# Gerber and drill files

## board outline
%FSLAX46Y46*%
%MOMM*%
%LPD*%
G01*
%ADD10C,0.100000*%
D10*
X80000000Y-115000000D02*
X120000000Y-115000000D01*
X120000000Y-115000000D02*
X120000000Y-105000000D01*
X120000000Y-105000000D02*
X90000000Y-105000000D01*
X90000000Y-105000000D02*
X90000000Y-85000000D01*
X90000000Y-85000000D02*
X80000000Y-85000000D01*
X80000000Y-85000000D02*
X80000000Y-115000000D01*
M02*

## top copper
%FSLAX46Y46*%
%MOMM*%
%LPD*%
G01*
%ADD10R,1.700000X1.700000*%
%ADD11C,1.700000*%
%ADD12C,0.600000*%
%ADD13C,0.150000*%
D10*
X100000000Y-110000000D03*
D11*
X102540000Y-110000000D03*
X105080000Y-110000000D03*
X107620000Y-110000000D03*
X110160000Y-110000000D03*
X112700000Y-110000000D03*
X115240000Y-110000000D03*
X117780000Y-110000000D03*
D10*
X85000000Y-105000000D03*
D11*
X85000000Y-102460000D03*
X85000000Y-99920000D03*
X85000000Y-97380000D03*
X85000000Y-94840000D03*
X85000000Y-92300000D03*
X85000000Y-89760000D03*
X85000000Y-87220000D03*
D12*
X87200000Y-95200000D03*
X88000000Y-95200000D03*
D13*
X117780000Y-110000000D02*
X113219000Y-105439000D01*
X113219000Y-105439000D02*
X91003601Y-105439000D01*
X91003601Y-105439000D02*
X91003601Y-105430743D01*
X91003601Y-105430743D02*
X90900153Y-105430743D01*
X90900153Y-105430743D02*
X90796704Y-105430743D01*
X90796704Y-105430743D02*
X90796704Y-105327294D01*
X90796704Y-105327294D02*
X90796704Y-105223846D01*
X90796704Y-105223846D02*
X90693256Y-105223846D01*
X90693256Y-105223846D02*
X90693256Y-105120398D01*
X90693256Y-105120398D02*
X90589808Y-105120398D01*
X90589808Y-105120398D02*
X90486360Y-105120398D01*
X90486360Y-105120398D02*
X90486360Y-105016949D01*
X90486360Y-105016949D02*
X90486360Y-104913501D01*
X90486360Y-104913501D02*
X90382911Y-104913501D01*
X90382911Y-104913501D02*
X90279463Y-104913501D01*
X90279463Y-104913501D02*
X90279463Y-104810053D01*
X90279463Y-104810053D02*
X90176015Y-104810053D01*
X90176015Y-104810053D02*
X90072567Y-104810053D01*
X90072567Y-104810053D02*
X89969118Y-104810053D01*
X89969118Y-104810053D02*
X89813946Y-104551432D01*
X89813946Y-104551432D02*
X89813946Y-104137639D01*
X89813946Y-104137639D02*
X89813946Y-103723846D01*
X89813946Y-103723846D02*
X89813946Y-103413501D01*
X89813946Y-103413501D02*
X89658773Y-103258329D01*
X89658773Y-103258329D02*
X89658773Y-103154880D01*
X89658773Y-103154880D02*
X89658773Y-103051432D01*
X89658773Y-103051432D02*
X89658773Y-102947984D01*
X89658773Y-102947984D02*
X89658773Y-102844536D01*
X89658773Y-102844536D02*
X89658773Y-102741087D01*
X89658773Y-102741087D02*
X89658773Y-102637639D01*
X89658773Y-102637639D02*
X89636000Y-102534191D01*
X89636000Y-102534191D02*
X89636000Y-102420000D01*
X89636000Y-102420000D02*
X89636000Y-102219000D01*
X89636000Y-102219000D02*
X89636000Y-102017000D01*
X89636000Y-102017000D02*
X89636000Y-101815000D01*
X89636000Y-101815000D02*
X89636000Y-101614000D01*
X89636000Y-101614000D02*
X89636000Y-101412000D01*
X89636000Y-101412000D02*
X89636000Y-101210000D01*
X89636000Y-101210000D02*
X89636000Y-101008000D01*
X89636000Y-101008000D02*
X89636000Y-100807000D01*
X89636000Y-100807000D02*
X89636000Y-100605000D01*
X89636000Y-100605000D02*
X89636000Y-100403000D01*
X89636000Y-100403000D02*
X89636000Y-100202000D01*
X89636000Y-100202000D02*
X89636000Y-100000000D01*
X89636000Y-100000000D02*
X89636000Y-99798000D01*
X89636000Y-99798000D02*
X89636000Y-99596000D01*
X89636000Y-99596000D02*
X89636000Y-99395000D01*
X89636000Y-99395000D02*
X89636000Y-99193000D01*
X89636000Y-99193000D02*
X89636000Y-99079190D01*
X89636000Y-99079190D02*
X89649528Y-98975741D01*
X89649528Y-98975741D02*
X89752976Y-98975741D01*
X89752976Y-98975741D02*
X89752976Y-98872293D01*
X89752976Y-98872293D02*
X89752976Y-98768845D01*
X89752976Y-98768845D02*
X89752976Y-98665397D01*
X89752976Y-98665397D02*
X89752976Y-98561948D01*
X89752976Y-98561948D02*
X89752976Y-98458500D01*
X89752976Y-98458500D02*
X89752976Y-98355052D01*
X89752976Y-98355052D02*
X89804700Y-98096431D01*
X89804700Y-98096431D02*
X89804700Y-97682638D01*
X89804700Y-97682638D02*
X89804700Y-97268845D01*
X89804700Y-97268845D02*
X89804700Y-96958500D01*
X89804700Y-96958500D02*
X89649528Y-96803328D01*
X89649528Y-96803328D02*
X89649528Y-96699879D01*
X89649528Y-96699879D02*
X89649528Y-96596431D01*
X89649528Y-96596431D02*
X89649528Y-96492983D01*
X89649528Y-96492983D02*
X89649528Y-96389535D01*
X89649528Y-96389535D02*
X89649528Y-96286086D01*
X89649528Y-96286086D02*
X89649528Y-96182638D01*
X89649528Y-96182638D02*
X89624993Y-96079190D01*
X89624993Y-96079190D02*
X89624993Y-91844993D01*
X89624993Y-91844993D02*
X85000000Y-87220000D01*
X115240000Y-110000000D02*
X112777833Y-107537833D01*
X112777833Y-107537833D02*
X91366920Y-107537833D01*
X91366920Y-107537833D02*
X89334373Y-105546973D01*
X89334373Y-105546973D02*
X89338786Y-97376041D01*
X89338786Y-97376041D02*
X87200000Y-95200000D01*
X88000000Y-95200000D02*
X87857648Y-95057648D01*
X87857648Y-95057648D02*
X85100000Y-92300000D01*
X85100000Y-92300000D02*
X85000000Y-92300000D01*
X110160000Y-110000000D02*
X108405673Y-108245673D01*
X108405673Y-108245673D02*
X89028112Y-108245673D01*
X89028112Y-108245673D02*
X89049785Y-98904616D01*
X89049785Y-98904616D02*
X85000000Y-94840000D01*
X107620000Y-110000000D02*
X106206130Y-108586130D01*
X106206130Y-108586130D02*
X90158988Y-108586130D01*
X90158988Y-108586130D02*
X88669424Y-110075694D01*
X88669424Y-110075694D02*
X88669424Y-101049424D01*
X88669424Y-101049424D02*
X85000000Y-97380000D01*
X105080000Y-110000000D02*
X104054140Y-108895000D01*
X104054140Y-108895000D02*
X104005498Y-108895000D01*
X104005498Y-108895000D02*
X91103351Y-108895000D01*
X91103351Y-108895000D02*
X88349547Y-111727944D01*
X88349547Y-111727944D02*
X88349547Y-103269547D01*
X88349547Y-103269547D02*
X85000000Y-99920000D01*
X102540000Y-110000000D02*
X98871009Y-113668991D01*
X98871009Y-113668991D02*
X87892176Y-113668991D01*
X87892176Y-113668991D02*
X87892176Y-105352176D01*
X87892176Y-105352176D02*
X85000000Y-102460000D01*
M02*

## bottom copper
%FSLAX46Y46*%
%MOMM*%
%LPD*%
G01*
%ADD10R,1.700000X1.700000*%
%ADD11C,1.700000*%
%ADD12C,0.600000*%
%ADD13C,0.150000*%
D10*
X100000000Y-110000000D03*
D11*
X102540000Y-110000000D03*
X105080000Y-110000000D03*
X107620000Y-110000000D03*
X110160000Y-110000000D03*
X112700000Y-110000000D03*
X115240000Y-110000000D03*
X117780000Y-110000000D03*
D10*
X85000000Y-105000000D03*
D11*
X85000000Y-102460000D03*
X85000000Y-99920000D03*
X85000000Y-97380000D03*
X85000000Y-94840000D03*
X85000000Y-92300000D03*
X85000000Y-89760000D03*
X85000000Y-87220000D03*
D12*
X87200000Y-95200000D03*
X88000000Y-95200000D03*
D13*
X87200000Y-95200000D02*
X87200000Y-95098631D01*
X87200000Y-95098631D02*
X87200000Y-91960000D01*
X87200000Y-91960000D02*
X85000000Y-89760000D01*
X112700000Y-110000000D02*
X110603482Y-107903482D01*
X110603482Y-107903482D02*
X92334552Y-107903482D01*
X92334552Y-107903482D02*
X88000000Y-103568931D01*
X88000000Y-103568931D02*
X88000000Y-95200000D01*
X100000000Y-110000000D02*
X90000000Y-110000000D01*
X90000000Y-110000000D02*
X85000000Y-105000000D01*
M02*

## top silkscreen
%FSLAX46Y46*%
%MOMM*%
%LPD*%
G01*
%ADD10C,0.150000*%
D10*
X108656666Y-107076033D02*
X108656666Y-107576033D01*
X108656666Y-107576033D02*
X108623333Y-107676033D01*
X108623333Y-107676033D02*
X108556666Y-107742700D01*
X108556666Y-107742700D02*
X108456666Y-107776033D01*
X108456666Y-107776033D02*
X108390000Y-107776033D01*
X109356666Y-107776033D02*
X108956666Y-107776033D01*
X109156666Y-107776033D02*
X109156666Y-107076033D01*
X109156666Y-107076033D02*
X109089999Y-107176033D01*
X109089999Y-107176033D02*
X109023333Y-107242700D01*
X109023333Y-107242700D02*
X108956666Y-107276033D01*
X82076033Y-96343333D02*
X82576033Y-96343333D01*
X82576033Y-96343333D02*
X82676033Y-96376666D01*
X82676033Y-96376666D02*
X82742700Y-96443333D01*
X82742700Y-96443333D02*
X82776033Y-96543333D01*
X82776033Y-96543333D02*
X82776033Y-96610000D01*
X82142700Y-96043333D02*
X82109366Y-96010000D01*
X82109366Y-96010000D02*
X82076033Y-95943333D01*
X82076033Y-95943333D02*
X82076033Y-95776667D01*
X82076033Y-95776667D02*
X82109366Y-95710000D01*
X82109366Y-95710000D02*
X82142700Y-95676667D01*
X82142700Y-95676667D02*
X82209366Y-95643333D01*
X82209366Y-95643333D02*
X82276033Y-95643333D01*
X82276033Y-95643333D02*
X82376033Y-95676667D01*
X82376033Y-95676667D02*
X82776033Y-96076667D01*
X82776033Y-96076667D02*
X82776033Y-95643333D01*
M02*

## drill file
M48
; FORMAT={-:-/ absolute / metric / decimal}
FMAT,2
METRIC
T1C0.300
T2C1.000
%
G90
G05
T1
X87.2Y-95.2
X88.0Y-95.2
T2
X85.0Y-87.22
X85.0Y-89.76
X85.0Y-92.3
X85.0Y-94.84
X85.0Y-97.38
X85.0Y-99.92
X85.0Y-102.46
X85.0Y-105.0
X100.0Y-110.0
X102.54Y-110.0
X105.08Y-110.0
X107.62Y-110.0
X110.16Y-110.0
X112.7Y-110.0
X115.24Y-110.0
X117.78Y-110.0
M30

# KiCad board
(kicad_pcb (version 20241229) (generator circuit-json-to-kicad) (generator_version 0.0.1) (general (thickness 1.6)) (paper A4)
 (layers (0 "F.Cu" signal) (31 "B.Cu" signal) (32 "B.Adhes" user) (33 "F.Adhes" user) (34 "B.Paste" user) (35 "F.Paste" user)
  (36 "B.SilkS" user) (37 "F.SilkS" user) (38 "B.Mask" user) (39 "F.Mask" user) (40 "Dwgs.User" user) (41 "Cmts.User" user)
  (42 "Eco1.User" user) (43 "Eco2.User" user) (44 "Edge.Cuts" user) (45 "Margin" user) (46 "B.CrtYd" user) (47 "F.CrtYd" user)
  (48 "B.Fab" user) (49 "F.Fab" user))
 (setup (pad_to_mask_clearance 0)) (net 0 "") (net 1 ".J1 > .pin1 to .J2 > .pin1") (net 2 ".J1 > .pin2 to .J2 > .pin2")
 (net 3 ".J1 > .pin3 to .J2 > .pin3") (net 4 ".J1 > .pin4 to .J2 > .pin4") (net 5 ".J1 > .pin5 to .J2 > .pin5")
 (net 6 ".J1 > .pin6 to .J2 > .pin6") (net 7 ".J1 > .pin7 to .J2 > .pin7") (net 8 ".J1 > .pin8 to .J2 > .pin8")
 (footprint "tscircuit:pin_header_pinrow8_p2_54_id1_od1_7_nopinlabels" (layer F.Cu) (at 108.89 110 0)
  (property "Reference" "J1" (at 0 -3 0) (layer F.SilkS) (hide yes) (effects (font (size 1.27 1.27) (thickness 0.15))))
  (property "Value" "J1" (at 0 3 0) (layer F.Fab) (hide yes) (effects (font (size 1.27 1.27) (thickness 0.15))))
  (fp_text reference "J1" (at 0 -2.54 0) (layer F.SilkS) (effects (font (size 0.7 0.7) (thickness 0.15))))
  (pad "1" thru_hole rect (at -8.89 0 0) (size 1.7 1.7) (drill 1) (layers *.Cu *.Mask) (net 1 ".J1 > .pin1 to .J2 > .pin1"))
  (pad "2" thru_hole circle (at -6.3500000000000005 0 0) (size 1.7 1.7) (drill 1) (layers *.Cu *.Mask) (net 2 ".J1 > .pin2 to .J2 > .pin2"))
  (pad "3" thru_hole circle (at -3.8100000000000005 0 0) (size 1.7 1.7) (drill 1) (layers *.Cu *.Mask) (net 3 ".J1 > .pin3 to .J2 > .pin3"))
  (pad "4" thru_hole circle (at -1.2700000000000005 0 0) (size 1.7 1.7) (drill 1) (layers *.Cu *.Mask) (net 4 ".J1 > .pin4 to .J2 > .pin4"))
  (pad "5" thru_hole circle (at 1.2699999999999996 0 0) (size 1.7 1.7) (drill 1) (layers *.Cu *.Mask) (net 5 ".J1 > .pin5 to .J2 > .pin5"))
  (pad "6" thru_hole circle (at 3.8099999999999987 0 0) (size 1.7 1.7) (drill 1) (layers *.Cu *.Mask) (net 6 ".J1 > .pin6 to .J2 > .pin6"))
  (pad "7" thru_hole circle (at 6.35 0 0) (size 1.7 1.7) (drill 1) (layers *.Cu *.Mask) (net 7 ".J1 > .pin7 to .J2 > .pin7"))
  (pad "8" thru_hole circle (at 8.89 0 0) (size 1.7 1.7) (drill 1) (layers *.Cu *.Mask) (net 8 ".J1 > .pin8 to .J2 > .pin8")))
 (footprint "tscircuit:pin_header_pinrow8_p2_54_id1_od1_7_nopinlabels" (layer F.Cu) (at 85 96.11 90)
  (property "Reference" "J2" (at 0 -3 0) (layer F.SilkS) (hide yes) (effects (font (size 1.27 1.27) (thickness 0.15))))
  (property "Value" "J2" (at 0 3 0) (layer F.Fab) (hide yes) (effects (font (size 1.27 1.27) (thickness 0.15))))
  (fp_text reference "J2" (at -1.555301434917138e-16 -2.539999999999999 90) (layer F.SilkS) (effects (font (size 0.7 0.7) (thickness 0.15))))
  (pad "1" thru_hole rect (at -8.89 5.443555022209985e-16 90) (size 1.7 1.7) (drill 1) (layers *.Cu *.Mask)
   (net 1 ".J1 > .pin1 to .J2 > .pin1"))
  (pad "2" thru_hole circle (at -6.3500000000000005 3.8882535872928466e-16 0) (size 1.7 1.7) (drill 1) (layers *.Cu *.Mask)
   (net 2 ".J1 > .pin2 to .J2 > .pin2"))
  (pad "3" thru_hole circle (at -3.8100000000000005 2.332952152375708e-16 0) (size 1.7 1.7) (drill 1) (layers *.Cu *.Mask)
   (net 3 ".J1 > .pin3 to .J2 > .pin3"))
  (pad "4" thru_hole circle (at -1.2700000000000005 7.776507174585695e-17 0) (size 1.7 1.7) (drill 1) (layers *.Cu *.Mask)
   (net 4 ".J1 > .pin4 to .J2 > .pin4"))
  (pad "5" thru_hole circle (at 1.2699999999999996 -7.77650717458569e-17 0) (size 1.7 1.7) (drill 1) (layers *.Cu *.Mask)
   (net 5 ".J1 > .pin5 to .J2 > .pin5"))
  (pad "6" thru_hole circle (at 3.8099999999999987 -2.3329521523757073e-16 0) (size 1.7 1.7) (drill 1) (layers *.Cu *.Mask)
   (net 6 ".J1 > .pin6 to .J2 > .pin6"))
  (pad "7" thru_hole circle (at 6.35 -3.888253587292846e-16 0) (size 1.7 1.7) (drill 1) (layers *.Cu *.Mask)
   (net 7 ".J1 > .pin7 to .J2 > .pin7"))
  (pad "8" thru_hole circle (at 8.89 -5.443555022209985e-16 0) (size 1.7 1.7) (drill 1) (layers *.Cu *.Mask)
   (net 8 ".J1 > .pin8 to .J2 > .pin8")))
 (segment (start 117.78 110) (end 113.219 105.439) (width 0.15) (layer F.Cu) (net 8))
 (segment (start 113.219 105.439) (end 91.00360101307515 105.439) (width 0.15) (layer F.Cu) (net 8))
 (segment (start 91.00360101307515 105.439) (end 91.00360101307515 105.43074251937742) (width 0.15) (layer F.Cu) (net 8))
 (segment (start 91.00360101307515 105.43074251937742) (end 90.90015273721309 105.43074251937742) (width 0.15) (layer F.Cu) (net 8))
 (segment (start 90.90015273721309 105.43074251937742) (end 90.79670446135103 105.43074251937742) (width 0.15) (layer F.Cu) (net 8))
 (segment (start 90.79670446135103 105.43074251937742) (end 90.79670446135103 105.32729424351534) (width 0.15) (layer F.Cu) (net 8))
 (segment (start 90.79670446135103 105.32729424351534) (end 90.79670446135103 105.22384596765328) (width 0.15) (layer F.Cu) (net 8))
 (segment (start 90.79670446135103 105.22384596765328) (end 90.69325618548895 105.22384596765328) (width 0.15) (layer F.Cu) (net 8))
 (segment (start 90.69325618548895 105.22384596765328) (end 90.69325618548895 105.12039769179121) (width 0.15) (layer F.Cu) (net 8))
 (segment (start 90.69325618548895 105.12039769179121) (end 90.58980790962688 105.12039769179121) (width 0.15) (layer F.Cu) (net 8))
 (segment (start 90.58980790962688 105.12039769179121) (end 90.4863596337648 105.12039769179121) (width 0.15) (layer F.Cu) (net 8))
 (segment (start 90.4863596337648 105.12039769179121) (end 90.4863596337648 105.01694941592913) (width 0.15) (layer F.Cu) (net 8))
 (segment (start 90.4863596337648 105.01694941592913) (end 90.4863596337648 104.91350114006707) (width 0.15) (layer F.Cu) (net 8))
 (segment (start 90.4863596337648 104.91350114006707) (end 90.38291135790274 104.91350114006707) (width 0.15) (layer F.Cu) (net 8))
 (segment (start 90.38291135790274 104.91350114006707) (end 90.27946308204068 104.91350114006707) (width 0.15) (layer F.Cu) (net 8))
 (segment (start 90.27946308204068 104.91350114006707) (end 90.27946308204068 104.810052864205) (width 0.15) (layer F.Cu) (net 8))
 (segment (start 90.27946308204068 104.810052864205) (end 90.1760148061786 104.810052864205) (width 0.15) (layer F.Cu) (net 8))
 (segment (start 90.1760148061786 104.810052864205) (end 90.07256653031654 104.810052864205) (width 0.15) (layer F.Cu) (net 8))
 (segment (start 90.07256653031654 104.810052864205) (end 89.96911825445447 104.810052864205) (width 0.15) (layer F.Cu) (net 8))
 (segment (start 89.96911825445447 104.810052864205) (end 89.81394584066136 104.55143217454983) (width 0.15) (layer F.Cu) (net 8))
 (segment (start 89.81394584066136 104.55143217454983) (end 89.81394584066136 104.13763907110155) (width 0.15) (layer F.Cu) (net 8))
 (segment (start 89.81394584066136 104.13763907110155) (end 89.81394584066136 103.72384596765328) (width 0.15) (layer F.Cu) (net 8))
 (segment (start 89.81394584066136 103.72384596765328) (end 89.81394584066136 103.41350114006707) (width 0.15) (layer F.Cu) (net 8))
 (segment (start 89.81394584066136 103.41350114006707) (end 89.65877342686827 103.25832872627397) (width 0.15) (layer F.Cu) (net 8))
 (segment (start 89.65877342686827 103.25832872627397) (end 89.65877342686827 103.1548804504119) (width 0.15) (layer F.Cu) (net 8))
 (segment (start 89.65877342686827 103.1548804504119) (end 89.65877342686827 103.05143217454983) (width 0.15) (layer F.Cu) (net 8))
 (segment (start 89.65877342686827 103.05143217454983) (end 89.65877342686827 102.94798389868777) (width 0.15) (layer F.Cu) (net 8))
 (segment (start 89.65877342686827 102.94798389868777) (end 89.65877342686827 102.84453562282569) (width 0.15) (layer F.Cu) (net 8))
 (segment (start 89.65877342686827 102.84453562282569) (end 89.65877342686827 102.74108734696362) (width 0.15) (layer F.Cu) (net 8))
 (segment (start 89.65877342686827 102.74108734696362) (end 89.65877342686827 102.63763907110155) (width 0.15) (layer F.Cu) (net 8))
 (segment (start 89.65877342686827 102.63763907110155) (end 89.636 102.53419079523948) (width 0.15) (layer F.Cu) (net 8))
 (segment (start 89.636 102.53419079523948) (end 89.636 102.42) (width 0.15) (layer F.Cu) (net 8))
 (segment (start 89.636 102.42) (end 89.636 102.219) (width 0.15) (layer F.Cu) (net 8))
 (segment (start 89.636 102.219) (end 89.636 102.017) (width 0.15) (layer F.Cu) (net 8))
 (segment (start 89.636 102.017) (end 89.636 101.815) (width 0.15) (layer F.Cu) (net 8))
 (segment (start 89.636 101.815) (end 89.636 101.614) (width 0.15) (layer F.Cu) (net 8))
 (segment (start 89.636 101.614) (end 89.636 101.412) (width 0.15) (layer F.Cu) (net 8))
 (segment (start 89.636 101.412) (end 89.636 101.21) (width 0.15) (layer F.Cu) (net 8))
 (segment (start 89.636 101.21) (end 89.636 101.008) (width 0.15) (layer F.Cu) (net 8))
 (segment (start 89.636 101.008) (end 89.636 100.807) (width 0.15) (layer F.Cu) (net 8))
 (segment (start 89.636 100.807) (end 89.636 100.605) (width 0.15) (layer F.Cu) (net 8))
 (segment (start 89.636 100.605) (end 89.636 100.403) (width 0.15) (layer F.Cu) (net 8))
 (segment (start 89.636 100.403) (end 89.636 100.202) (width 0.15) (layer F.Cu) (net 8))
 (segment (start 89.636 100.202) (end 89.636 100) (width 0.15) (layer F.Cu) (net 8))
 (segment (start 89.636 100) (end 89.636 99.798) (width 0.15) (layer F.Cu) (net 8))
 (segment (start 89.636 99.798) (end 89.636 99.596) (width 0.15) (layer F.Cu) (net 8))
 (segment (start 89.636 99.596) (end 89.636 99.395) (width 0.15) (layer F.Cu) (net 8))
 (segment (start 89.636 99.395) (end 89.636 99.193) (width 0.15) (layer F.Cu) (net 8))
 (segment (start 89.636 99.193) (end 89.636 99.07918970210036) (width 0.15) (layer F.Cu) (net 8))
 (segment (start 89.636 99.07918970210036) (end 89.64952790927448 98.9757414262383) (width 0.15) (layer F.Cu) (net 8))
 (segment (start 89.64952790927448 98.9757414262383) (end 89.75297618513655 98.9757414262383) (width 0.15) (layer F.Cu) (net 8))
 (segment (start 89.75297618513655 98.9757414262383) (end 89.75297618513655 98.87229315037622) (width 0.15) (layer F.Cu) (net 8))
 (segment (start 89.75297618513655 98.87229315037622) (end 89.75297618513655 98.76884487451416) (width 0.15) (layer F.Cu) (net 8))
 (segment (start 89.75297618513655 98.76884487451416) (end 89.75297618513655 98.66539659865208) (width 0.15) (layer F.Cu) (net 8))
 (segment (start 89.75297618513655 98.66539659865208) (end 89.75297618513655 98.56194832279002) (width 0.15) (layer F.Cu) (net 8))
 (segment (start 89.75297618513655 98.56194832279002) (end 89.75297618513655 98.45850004692795) (width 0.15) (layer F.Cu) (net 8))
 (segment (start 89.75297618513655 98.45850004692795) (end 89.75297618513655 98.35505177106587) (width 0.15) (layer F.Cu) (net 8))
 (segment (start 89.75297618513655 98.35505177106587) (end 89.80470032306758 98.09643108141071) (width 0.15) (layer F.Cu) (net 8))
 (segment (start 89.80470032306758 98.09643108141071) (end 89.80470032306758 97.68263797796243) (width 0.15) (layer F.Cu) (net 8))
 (segment (start 89.80470032306758 97.68263797796243) (end 89.80470032306758 97.26884487451416) (width 0.15) (layer F.Cu) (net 8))
 (segment (start 89.80470032306758 97.26884487451416) (end 89.80470032306758 96.95850004692795) (width 0.15) (layer F.Cu) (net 8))
 (segment (start 89.80470032306758 96.95850004692795) (end 89.64952790927448 96.80332763313484) (width 0.15) (layer F.Cu) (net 8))
 (segment (start 89.64952790927448 96.80332763313484) (end 89.64952790927448 96.69987935727278) (width 0.15) (layer F.Cu) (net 8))
 (segment (start 89.64952790927448 96.69987935727278) (end 89.64952790927448 96.59643108141071) (width 0.15) (layer F.Cu) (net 8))
 (segment (start 89.64952790927448 96.59643108141071) (end 89.64952790927448 96.49298280554864) (width 0.15) (layer F.Cu) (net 8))
 (segment (start 89.64952790927448 96.49298280554864) (end 89.64952790927448 96.38953452968657) (width 0.15) (layer F.Cu) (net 8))
 (segment (start 89.64952790927448 96.38953452968657) (end 89.64952790927448 96.28608625382451) (width 0.15) (layer F.Cu) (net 8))
 (segment (start 89.64952790927448 96.28608625382451) (end 89.64952790927448 96.18263797796243) (width 0.15) (layer F.Cu) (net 8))
 (segment (start 89.64952790927448 96.18263797796243) (end 89.62499268844161 96.07918970210036) (width 0.15) (layer F.Cu) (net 8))
 (segment (start 89.62499268844161 96.07918970210036) (end 89.62499268844161 91.84499268844161) (width 0.15) (layer F.Cu) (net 8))
 (segment (start 89.62499268844161 91.84499268844161) (end 85 87.22) (width 0.15) (layer F.Cu) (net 8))
 (segment (start 115.24 110) (end 112.77783324481014 107.53783324481014) (width 0.15) (layer F.Cu) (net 7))
 (segment (start 112.77783324481014 107.53783324481014) (end 91.36692030316749 107.53783324481014) (width 0.15) (layer F.Cu) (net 7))
 (segment (start 91.36692030316749 107.53783324481014) (end 89.33437344650389 105.54697301333326) (width 0.15) (layer F.Cu) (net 7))
 (segment (start 89.33437344650389 105.54697301333326) (end 89.33878628174294 97.37604069813212) (width 0.15) (layer F.Cu) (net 7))
 (segment (start 89.33878628174294 97.37604069813212) (end 87.2 95.2) (width 0.15) (layer F.Cu) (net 7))
 (segment (start 87.2 95.2) (end 87.2 95.09863104739347) (width 0.15) (layer B.Cu) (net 7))
 (segment (start 87.2 95.09863104739347) (end 87.2 91.96) (width 0.15) (layer B.Cu) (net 7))
 (segment (start 87.2 91.96) (end 85 89.76) (width 0.15) (layer B.Cu) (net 7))
 (segment (start 112.7 110) (end 110.60348236580158 107.90348236580158) (width 0.15) (layer B.Cu) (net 6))
 (segment (start 110.60348236580158 107.90348236580158) (end 92.33455173037902 107.90348236580158) (width 0.15) (layer B.Cu) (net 6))
 (segment (start 92.33455173037902 107.90348236580158) (end 88 103.56893063542256) (width 0.15) (layer B.Cu) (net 6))
 (segment (start 88 103.56893063542256) (end 88 95.2) (width 0.15) (layer B.Cu) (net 6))
 (segment (start 88 95.2) (end 87.85764760102865 95.05764760102863) (width 0.15) (layer F.Cu) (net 6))
 (segment (start 87.85764760102865 95.05764760102863) (end 85.1 92.3) (width 0.15) (layer F.Cu) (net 6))
 (segment (start 85.1 92.3) (end 85 92.3) (width 0.15) (layer F.Cu) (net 6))
 (segment (start 110.16 110) (end 108.40567338036273 108.24567338036272) (width 0.15) (layer F.Cu) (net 5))
 (segment (start 108.40567338036273 108.24567338036272) (end 89.02811192644441 108.24567338036272) (width 0.15) (layer F.Cu) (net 5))
 (segment (start 89.02811192644441 108.24567338036272) (end 89.04978503151894 98.90461624668895) (width 0.15) (layer F.Cu) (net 5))
 (segment (start 89.04978503151894 98.90461624668895) (end 85 94.84) (width 0.15) (layer F.Cu) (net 5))
 (segment (start 107.62 110) (end 106.20613024048843 108.58613024048843) (width 0.15) (layer F.Cu) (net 4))
 (segment (start 106.20613024048843 108.58613024048843) (end 90.15898804054336 108.58613024048843) (width 0.15) (layer F.Cu) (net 4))
 (segment (start 90.15898804054336 108.58613024048843) (end 88.66942445956417 110.07569382146764) (width 0.15) (layer F.Cu) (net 4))
 (segment (start 88.66942445956417 110.07569382146764) (end 88.66942445956417 101.04942445956416) (width 0.15) (layer F.Cu) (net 4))
 (segment (start 88.66942445956417 101.04942445956416) (end 85 97.38) (width 0.15) (layer F.Cu) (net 4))
 (segment (start 105.08 110) (end 104.05413977259249 108.895) (width 0.15) (layer F.Cu) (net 3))
 (segment (start 104.05413977259249 108.895) (end 104.00549755734117 108.895) (width 0.15) (layer F.Cu) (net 3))
 (segment (start 104.00549755734117 108.895) (end 91.1033507815009 108.895) (width 0.15) (layer F.Cu) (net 3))
 (segment (start 91.1033507815009 108.895) (end 88.34954662570104 111.72794392839235) (width 0.15) (layer F.Cu) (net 3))
 (segment (start 88.34954662570104 111.72794392839235) (end 88.34954662570104 103.26954662570104) (width 0.15) (layer F.Cu) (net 3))
 (segment (start 88.34954662570104 103.26954662570104) (end 85 99.92) (width 0.15) (layer F.Cu) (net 3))
 (segment (start 102.54 110) (end 98.8710089430543 113.6689910569457) (width 0.15) (layer F.Cu) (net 2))
 (segment (start 98.8710089430543 113.6689910569457) (end 87.8921759286383 113.6689910569457) (width 0.15) (layer F.Cu) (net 2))
 (segment (start 87.8921759286383 113.6689910569457) (end 87.8921759286383 105.3521759286383) (width 0.15) (layer F.Cu) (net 2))
 (segment (start 87.8921759286383 105.3521759286383) (end 85 102.46) (width 0.15) (layer F.Cu) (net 2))
 (segment (start 100 110) (end 90 110) (width 0.15) (layer B.Cu) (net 1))
 (segment (start 90 110) (end 85 105) (width 0.15) (layer B.Cu) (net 1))
 (gr_line (start 80 115) (end 120 115) (width 0.1) (layer Edge.Cuts))
 (gr_line (start 120 115) (end 120 105) (width 0.1) (layer Edge.Cuts))
 (gr_line (start 120 105) (end 90 105) (width 0.1) (layer Edge.Cuts))
 (gr_line (start 90 105) (end 90 85) (width 0.1) (layer Edge.Cuts))
 (gr_line (start 90 85) (end 80 85) (width 0.1) (layer Edge.Cuts))
 (gr_line (start 80 85) (end 80 115) (width 0.1) (layer Edge.Cuts))
 (via (at 87.2 95.2) (size 0.6) (drill 0.3) (layers F.Cu B.Cu) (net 7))
 (via (at 88 95.2) (size 0.6) (drill 0.3) (layers F.Cu B.Cu) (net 6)))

